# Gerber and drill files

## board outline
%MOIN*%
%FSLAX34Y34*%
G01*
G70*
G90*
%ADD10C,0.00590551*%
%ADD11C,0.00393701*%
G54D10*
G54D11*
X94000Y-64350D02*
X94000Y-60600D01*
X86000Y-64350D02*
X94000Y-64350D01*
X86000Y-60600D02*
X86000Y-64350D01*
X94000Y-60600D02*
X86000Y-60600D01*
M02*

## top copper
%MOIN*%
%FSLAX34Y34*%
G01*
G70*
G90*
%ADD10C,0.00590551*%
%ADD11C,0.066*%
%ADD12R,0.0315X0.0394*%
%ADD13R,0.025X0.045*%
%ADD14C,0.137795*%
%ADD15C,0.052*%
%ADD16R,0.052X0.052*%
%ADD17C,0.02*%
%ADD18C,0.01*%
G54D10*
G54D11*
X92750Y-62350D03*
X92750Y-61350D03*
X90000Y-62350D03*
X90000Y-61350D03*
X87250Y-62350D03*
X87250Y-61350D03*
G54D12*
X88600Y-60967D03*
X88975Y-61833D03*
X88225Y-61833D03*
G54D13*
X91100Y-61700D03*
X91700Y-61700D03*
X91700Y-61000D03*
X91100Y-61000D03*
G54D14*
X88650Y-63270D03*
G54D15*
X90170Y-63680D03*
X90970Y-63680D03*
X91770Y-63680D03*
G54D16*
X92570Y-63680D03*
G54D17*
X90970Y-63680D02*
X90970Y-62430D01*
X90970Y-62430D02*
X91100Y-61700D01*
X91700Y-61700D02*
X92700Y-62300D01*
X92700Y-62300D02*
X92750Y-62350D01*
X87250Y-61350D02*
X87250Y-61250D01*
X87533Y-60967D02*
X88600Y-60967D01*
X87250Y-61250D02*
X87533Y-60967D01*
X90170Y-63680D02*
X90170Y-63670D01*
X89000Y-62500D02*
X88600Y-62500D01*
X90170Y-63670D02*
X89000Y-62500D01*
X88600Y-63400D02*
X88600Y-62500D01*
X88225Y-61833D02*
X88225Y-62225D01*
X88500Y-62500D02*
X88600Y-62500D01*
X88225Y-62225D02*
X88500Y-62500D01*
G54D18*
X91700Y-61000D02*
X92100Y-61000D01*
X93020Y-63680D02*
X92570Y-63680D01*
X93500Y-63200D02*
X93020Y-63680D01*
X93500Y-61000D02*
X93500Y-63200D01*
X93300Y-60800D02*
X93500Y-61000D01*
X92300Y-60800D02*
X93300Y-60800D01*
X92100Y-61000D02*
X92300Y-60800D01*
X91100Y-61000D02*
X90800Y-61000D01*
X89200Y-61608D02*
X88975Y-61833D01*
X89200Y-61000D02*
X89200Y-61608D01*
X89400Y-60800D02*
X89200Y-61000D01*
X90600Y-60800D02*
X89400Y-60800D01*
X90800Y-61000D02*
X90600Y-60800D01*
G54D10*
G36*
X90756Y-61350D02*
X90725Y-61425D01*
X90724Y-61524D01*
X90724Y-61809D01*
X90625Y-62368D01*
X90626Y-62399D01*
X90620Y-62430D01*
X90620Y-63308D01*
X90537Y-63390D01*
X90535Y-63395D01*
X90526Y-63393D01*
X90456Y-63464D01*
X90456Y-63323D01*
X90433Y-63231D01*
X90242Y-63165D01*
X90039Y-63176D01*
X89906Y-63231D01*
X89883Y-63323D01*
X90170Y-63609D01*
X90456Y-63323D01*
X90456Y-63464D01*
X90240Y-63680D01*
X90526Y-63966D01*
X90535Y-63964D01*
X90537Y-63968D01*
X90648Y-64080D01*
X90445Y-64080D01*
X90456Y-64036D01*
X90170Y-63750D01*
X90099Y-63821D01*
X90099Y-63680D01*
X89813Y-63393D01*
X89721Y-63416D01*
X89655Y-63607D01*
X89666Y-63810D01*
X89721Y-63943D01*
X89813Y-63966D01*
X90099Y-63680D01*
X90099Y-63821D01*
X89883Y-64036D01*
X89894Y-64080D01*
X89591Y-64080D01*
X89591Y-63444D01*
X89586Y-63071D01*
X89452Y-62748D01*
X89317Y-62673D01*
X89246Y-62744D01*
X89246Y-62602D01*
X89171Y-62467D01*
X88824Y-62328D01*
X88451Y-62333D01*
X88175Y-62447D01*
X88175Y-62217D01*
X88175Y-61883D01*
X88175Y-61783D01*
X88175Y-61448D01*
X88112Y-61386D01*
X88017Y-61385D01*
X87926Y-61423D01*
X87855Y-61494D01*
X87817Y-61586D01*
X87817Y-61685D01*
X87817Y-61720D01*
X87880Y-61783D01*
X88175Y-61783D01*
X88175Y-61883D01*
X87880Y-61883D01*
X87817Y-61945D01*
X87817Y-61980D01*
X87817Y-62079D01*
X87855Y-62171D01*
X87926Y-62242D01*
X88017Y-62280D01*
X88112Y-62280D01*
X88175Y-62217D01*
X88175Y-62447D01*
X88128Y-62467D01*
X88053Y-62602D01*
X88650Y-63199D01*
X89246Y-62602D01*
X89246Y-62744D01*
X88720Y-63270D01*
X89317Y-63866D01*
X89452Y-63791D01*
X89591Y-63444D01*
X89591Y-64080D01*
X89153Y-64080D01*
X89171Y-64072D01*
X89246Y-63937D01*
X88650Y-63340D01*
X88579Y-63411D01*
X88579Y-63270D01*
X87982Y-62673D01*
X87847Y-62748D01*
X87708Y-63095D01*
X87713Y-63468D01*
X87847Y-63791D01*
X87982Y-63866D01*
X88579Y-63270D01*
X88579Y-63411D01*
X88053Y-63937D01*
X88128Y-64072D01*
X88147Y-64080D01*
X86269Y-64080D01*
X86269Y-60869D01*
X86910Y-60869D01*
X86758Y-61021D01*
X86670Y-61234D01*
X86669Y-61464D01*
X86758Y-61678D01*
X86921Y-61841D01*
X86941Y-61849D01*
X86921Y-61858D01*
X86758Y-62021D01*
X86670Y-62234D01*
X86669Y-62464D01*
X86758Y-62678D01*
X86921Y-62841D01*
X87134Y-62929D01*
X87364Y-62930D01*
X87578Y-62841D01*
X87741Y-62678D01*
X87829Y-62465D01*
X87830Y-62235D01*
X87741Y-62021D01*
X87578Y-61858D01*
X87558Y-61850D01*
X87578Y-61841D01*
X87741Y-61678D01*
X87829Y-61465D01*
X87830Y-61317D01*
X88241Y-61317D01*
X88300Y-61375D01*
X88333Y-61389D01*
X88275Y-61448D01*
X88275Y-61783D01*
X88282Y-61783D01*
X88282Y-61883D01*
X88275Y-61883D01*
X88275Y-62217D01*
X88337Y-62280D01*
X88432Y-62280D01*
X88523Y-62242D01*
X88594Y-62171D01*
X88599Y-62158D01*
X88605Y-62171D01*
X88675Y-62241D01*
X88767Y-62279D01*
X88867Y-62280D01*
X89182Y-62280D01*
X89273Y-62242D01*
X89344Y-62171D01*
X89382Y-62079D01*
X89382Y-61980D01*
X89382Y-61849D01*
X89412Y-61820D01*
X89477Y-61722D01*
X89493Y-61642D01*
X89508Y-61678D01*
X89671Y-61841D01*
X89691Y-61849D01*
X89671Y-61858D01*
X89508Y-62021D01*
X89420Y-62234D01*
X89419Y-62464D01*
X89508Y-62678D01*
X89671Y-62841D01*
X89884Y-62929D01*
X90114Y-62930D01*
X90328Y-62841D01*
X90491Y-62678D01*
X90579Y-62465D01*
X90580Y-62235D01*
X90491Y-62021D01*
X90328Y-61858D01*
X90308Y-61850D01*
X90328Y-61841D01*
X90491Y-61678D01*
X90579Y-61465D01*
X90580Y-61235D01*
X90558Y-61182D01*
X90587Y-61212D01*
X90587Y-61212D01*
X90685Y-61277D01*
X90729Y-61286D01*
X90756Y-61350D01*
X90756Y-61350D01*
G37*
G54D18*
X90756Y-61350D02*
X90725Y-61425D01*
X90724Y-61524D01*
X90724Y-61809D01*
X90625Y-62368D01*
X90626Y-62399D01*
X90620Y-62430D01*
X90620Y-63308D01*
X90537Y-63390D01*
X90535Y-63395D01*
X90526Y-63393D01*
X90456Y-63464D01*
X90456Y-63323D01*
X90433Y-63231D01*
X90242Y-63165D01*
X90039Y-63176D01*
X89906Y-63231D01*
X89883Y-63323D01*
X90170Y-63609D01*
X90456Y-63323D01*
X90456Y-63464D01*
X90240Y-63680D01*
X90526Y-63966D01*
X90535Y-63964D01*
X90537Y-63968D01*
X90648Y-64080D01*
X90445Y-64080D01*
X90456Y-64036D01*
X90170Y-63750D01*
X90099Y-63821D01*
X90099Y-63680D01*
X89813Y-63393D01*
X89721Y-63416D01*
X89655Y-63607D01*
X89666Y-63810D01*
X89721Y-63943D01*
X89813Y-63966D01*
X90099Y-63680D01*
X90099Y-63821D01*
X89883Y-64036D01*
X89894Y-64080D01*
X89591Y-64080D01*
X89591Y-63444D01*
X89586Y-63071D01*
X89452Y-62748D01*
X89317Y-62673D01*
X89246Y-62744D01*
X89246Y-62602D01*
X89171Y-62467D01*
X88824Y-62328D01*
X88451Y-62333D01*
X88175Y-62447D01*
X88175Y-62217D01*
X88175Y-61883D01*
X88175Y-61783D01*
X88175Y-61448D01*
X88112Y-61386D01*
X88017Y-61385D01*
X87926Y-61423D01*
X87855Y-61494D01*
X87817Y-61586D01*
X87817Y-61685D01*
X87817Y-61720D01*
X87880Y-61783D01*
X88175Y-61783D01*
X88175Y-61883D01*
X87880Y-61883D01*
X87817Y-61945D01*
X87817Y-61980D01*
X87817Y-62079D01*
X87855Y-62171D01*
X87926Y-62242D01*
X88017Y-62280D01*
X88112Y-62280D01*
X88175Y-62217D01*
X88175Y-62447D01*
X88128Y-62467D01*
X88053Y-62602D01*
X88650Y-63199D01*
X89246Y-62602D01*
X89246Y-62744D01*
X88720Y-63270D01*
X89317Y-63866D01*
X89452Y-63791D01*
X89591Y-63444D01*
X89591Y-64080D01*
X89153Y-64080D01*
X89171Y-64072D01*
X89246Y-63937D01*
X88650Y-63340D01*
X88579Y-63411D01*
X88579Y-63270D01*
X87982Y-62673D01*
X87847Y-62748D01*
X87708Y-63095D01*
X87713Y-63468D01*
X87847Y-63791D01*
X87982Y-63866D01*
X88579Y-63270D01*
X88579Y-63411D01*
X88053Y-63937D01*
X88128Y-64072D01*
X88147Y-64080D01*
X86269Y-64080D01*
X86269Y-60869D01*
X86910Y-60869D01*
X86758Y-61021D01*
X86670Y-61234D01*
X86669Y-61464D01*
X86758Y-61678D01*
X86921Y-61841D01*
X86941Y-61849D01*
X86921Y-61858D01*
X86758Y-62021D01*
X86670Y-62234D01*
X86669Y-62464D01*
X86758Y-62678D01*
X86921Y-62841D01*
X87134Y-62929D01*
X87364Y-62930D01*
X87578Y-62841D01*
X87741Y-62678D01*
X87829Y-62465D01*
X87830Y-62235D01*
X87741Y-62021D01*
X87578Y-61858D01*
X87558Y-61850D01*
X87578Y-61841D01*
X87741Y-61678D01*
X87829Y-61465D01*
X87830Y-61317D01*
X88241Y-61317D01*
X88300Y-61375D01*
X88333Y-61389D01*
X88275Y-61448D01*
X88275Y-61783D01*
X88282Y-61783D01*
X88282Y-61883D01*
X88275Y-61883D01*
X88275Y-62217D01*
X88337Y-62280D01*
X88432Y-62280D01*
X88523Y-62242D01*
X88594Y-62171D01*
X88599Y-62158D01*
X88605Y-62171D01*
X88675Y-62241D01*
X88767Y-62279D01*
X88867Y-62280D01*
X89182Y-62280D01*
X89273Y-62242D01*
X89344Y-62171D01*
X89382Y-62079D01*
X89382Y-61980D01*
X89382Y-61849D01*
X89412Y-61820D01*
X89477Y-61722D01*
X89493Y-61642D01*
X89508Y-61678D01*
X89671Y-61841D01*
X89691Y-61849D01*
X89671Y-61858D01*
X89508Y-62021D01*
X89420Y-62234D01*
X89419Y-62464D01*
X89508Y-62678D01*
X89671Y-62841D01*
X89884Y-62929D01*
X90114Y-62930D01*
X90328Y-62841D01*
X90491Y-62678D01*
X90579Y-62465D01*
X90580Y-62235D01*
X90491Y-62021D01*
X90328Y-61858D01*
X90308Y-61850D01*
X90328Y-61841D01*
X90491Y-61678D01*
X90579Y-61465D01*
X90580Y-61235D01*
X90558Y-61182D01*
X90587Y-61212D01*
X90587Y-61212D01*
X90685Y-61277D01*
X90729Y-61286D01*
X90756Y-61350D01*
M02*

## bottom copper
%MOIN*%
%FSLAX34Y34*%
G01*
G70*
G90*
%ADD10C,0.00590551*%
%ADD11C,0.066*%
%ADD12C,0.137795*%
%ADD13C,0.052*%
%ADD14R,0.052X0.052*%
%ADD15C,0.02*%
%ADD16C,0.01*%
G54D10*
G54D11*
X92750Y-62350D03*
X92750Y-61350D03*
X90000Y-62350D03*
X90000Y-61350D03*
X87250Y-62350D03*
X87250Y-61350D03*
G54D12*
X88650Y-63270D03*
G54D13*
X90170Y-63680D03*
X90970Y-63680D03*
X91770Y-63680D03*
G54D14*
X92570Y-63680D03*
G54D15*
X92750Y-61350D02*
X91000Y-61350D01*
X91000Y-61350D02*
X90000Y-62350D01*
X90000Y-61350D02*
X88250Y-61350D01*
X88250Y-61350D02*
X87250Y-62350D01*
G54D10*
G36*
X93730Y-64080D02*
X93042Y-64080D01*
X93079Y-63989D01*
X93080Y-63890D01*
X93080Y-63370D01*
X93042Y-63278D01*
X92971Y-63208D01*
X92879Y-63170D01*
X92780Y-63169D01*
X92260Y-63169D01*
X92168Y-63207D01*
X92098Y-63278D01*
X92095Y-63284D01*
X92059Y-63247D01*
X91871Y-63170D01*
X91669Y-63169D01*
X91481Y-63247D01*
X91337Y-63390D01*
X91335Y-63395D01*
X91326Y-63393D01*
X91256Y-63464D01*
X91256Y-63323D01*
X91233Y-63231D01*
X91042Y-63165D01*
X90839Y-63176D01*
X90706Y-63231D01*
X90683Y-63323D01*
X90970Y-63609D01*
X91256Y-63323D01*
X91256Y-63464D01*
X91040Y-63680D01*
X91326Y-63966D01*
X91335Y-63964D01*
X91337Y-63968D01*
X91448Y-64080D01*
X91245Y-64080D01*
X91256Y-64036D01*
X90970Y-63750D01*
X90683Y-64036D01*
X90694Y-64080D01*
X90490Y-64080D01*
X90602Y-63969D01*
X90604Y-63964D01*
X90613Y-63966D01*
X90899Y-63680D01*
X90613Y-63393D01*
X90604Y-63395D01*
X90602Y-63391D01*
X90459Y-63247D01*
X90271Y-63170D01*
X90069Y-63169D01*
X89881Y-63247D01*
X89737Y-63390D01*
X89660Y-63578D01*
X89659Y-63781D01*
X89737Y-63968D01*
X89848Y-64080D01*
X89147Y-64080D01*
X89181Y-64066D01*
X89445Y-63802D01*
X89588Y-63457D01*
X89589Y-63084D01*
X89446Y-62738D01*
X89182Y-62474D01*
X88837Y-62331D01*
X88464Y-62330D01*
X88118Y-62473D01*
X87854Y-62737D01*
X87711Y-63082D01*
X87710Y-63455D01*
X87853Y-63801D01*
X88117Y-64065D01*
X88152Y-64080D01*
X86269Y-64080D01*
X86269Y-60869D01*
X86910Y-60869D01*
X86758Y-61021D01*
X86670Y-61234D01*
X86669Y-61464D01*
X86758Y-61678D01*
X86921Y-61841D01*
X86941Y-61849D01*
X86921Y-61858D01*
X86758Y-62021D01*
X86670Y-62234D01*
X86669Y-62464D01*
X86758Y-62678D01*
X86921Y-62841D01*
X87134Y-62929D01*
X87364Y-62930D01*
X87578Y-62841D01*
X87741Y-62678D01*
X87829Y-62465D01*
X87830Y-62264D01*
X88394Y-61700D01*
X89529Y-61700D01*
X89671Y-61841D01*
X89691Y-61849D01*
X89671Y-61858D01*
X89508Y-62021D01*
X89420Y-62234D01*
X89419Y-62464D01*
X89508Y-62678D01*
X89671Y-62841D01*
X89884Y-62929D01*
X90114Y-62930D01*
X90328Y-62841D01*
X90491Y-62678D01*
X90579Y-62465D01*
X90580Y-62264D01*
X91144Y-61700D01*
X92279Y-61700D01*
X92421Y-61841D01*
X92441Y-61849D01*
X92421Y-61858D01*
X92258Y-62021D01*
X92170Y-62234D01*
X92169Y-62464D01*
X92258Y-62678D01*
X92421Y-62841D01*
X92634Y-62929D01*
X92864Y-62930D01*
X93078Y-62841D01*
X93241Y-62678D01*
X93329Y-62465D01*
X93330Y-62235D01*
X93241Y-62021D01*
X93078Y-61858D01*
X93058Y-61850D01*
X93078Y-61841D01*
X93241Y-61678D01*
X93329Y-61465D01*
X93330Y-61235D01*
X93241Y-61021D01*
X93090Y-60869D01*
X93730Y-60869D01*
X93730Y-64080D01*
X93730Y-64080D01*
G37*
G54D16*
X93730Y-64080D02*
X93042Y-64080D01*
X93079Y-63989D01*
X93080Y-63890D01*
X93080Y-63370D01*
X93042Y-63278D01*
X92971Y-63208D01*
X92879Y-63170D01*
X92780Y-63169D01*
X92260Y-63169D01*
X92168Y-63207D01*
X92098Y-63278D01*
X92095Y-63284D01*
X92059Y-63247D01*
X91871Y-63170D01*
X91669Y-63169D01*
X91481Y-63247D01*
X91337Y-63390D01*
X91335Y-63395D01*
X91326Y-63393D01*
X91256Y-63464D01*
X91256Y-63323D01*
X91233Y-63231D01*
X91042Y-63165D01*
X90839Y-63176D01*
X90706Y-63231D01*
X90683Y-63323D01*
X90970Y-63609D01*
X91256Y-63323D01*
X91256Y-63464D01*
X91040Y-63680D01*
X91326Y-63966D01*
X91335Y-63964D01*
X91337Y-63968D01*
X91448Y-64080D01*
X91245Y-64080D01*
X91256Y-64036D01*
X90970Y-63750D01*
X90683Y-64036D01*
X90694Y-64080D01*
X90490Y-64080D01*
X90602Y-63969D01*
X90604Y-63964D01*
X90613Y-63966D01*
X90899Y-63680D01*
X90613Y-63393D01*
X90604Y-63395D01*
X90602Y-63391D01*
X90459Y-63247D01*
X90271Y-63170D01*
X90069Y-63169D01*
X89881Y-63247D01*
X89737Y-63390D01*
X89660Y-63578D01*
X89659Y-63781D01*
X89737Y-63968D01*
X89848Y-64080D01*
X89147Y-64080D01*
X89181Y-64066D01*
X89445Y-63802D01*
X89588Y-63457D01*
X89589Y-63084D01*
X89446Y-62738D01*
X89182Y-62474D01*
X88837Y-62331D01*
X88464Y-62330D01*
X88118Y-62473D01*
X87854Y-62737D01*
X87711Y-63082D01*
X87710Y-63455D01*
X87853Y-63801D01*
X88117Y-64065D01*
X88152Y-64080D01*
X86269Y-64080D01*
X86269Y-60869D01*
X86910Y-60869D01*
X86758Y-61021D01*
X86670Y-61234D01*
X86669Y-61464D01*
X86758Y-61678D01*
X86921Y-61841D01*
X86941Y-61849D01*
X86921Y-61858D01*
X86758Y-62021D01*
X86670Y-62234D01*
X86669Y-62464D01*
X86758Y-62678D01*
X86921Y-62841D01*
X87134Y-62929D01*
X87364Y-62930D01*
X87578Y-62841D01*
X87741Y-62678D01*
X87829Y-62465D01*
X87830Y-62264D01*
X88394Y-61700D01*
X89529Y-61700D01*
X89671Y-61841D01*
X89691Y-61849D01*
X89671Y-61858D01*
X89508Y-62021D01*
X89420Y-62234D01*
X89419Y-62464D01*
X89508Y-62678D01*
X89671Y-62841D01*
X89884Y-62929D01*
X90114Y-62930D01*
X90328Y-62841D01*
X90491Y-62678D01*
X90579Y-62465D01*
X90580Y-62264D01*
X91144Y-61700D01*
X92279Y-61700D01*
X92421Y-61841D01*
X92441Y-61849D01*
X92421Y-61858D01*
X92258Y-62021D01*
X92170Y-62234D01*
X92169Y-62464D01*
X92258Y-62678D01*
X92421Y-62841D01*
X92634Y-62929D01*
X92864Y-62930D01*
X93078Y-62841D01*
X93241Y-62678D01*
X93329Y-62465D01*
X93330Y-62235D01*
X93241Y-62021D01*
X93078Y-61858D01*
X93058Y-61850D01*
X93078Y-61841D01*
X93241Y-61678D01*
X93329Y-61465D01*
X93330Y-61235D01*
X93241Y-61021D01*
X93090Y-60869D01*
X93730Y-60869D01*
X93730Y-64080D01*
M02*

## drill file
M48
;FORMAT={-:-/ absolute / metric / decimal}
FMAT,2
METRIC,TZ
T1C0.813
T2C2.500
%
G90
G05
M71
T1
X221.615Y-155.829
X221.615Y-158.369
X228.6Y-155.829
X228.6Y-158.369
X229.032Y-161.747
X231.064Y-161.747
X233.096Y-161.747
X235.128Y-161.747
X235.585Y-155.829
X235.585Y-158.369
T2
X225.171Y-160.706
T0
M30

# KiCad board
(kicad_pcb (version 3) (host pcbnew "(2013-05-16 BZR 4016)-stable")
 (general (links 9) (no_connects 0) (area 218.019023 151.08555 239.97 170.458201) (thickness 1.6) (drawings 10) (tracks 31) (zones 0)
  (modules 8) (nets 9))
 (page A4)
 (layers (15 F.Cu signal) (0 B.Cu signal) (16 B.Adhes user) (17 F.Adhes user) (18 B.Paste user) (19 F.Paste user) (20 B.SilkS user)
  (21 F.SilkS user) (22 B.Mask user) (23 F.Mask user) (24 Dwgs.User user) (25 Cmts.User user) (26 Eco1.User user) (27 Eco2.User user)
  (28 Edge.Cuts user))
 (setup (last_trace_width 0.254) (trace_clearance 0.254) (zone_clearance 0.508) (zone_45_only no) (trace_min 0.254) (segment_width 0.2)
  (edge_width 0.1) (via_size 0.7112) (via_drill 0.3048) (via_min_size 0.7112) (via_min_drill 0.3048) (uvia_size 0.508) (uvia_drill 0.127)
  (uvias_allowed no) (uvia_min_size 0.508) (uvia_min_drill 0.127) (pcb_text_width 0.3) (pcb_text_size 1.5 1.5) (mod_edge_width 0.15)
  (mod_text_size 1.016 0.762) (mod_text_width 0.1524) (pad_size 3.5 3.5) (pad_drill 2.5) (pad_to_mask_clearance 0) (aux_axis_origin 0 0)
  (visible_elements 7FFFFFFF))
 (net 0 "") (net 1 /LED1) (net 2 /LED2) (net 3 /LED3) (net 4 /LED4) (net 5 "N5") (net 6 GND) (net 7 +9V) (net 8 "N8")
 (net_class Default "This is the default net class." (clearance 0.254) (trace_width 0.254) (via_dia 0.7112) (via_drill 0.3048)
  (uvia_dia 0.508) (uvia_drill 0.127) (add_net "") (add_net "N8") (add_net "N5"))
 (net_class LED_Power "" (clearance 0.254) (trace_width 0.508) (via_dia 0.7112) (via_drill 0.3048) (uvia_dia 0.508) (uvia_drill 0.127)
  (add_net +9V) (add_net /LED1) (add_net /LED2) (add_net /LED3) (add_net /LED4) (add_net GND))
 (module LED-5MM (layer B.Cu) (at 235.585 157.099 90)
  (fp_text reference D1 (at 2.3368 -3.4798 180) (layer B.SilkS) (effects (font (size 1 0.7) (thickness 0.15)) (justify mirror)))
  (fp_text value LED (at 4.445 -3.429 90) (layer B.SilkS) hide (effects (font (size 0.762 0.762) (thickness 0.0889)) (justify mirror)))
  (pad 1 thru_hole circle (at -1.27 0 90) (size 1.6764 1.6764) (drill 0.8128) (layers *.Cu *.Mask B.SilkS) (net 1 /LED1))
  (pad 2 thru_hole circle (at 1.27 0 90) (size 1.6764 1.6764) (drill 0.8128) (layers *.Cu *.Mask B.SilkS) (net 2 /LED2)))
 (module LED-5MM (layer B.Cu) (at 228.6 157.099 90)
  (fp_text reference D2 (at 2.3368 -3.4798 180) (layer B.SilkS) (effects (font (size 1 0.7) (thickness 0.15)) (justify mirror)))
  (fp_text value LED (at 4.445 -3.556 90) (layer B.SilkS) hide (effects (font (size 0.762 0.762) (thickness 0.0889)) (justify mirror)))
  (pad 1 thru_hole circle (at -1.27 0 90) (size 1.6764 1.6764) (drill 0.8128) (layers *.Cu *.Mask B.SilkS) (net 2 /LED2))
  (pad 2 thru_hole circle (at 1.27 0 90) (size 1.6764 1.6764) (drill 0.8128) (layers *.Cu *.Mask B.SilkS) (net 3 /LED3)))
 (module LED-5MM (layer B.Cu) (at 221.615 157.099 90)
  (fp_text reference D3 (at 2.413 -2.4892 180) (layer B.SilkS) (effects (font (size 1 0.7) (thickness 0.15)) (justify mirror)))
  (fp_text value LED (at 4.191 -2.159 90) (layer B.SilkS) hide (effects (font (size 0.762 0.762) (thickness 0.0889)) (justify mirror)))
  (pad 1 thru_hole circle (at -1.27 0 90) (size 1.6764 1.6764) (drill 0.8128) (layers *.Cu *.Mask B.SilkS) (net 3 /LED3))
  (pad 2 thru_hole circle (at 1.27 0 90) (size 1.6764 1.6764) (drill 0.8128) (layers *.Cu *.Mask B.SilkS) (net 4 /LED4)))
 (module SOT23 (layer F.Cu) (at 225.044 155.956)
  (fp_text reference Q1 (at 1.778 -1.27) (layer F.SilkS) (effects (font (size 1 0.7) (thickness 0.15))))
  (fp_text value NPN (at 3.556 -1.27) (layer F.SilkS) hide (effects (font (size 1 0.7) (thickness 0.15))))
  (pad 3 smd rect (at 0 -1.09982) (size 0.8001 1.00076) (layers F.Cu F.Paste F.Mask) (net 4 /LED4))
  (pad 2 smd rect (at 0.9525 1.09982) (size 0.8001 1.00076) (layers F.Cu F.Paste F.Mask) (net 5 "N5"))
  (pad 1 smd rect (at -0.9525 1.09982) (size 0.8001 1.00076) (layers F.Cu F.Paste F.Mask) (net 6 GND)))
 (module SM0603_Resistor (layer F.Cu) (at 232.156 156.718)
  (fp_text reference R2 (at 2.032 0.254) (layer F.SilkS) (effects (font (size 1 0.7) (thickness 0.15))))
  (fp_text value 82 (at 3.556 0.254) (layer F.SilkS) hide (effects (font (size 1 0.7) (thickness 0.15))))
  (pad 1 smd rect (at -0.762 0) (size 0.635 1.143) (layers F.Cu F.Paste F.Mask) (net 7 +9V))
  (pad 2 smd rect (at 0.762 0) (size 0.635 1.143) (layers F.Cu F.Paste F.Mask) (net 1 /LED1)))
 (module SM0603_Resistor (layer F.Cu) (at 232.156 154.94 180)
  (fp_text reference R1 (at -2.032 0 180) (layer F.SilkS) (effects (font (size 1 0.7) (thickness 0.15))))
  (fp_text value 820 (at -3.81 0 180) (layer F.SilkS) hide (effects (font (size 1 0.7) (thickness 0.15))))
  (pad 1 smd rect (at -0.762 0 180) (size 0.635 1.143) (layers F.Cu F.Paste F.Mask) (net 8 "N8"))
  (pad 2 smd rect (at 0.762 0 180) (size 0.635 1.143) (layers F.Cu F.Paste F.Mask) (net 5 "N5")))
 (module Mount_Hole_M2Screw (layer F.Cu) (at 225.171 160.7058)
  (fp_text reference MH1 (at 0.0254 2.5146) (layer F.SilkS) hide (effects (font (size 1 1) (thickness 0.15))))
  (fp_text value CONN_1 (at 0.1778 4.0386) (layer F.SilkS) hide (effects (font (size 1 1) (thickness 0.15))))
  (pad 1 thru_hole circle (at 0 0) (size 3.5 3.5) (drill 2.5) (layers *.Cu *.Mask F.SilkS) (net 6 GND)))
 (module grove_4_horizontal (layer F.Cu) (at 227.076 160.274 90)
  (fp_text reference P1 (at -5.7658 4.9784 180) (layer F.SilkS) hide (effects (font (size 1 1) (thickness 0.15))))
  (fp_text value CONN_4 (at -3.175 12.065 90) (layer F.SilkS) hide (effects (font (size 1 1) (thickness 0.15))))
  (pad 4 thru_hole circle (at -1.4732 1.9558 90) (size 1.3208 1.3208) (drill 0.8128) (layers *.Cu *.Mask F.SilkS) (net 6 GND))
  (pad 3 thru_hole circle (at -1.4732 3.9878 90) (size 1.3208 1.3208) (drill 0.8128) (layers *.Cu *.Mask F.SilkS) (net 7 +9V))
  (pad 2 thru_hole circle (at -1.4732 6.0198 90) (size 1.3208 1.3208) (drill 0.8128) (layers *.Cu *.Mask F.SilkS))
  (pad 1 thru_hole rect (at -1.4732 8.0518 90) (size 1.3208 1.3208) (drill 0.8128) (layers *.Cu *.Mask F.SilkS) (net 8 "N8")))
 (gr_line (start 238.76 163.449) (end 238.76 153.924) (angle 90) (layer Edge.Cuts) (width 0.1))
 (gr_line (start 218.44 163.449) (end 238.76 163.449) (angle 90) (layer Edge.Cuts) (width 0.1))
 (gr_line (start 218.44 153.924) (end 218.44 163.449) (angle 90) (layer Edge.Cuts) (width 0.1))
 (gr_line (start 238.76 153.924) (end 218.44 153.924) (angle 90) (layer Edge.Cuts) (width 0.1))
 (segment (start 231.0638 161.7472) (end 231.0638 158.5722) (width 0.508) (layer F.Cu) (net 7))
 (segment (start 231.0638 158.5722) (end 231.394 156.718) (width 0.508) (layer F.Cu) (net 7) (status 20))
 (segment (start 232.918 156.718) (end 235.458 158.242) (width 0.508) (layer F.Cu) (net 1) (status 10))
 (segment (start 235.458 158.242) (end 235.585 158.369) (width 0.508) (layer F.Cu) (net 1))
 (segment (start 235.585 155.829) (end 231.14 155.829) (width 0.508) (layer B.Cu) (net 2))
 (segment (start 231.14 155.829) (end 228.6 158.369) (width 0.508) (layer B.Cu) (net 2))
 (segment (start 228.6 155.829) (end 224.155 155.829) (width 0.508) (layer B.Cu) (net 3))
 (segment (start 224.155 155.829) (end 221.615 158.369) (width 0.508) (layer B.Cu) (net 3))
 (segment (start 221.615 155.829) (end 221.615 155.575) (width 0.508) (layer F.Cu) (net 4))
 (segment (start 222.33382 154.85618) (end 225.044 154.85618) (width 0.508) (layer F.Cu) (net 4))
 (segment (start 221.615 155.575) (end 222.33382 154.85618) (width 0.508) (layer F.Cu) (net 4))
 (segment (start 229.0318 161.7472) (end 229.0318 161.7218) (width 0.508) (layer F.Cu) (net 6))
 (segment (start 226.06 158.75) (end 225.044 158.75) (width 0.508) (layer F.Cu) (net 6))
 (segment (start 229.0318 161.7218) (end 226.06 158.75) (width 0.508) (layer F.Cu) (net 6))
 (segment (start 225.044 161.036) (end 225.044 158.75) (width 0.508) (layer F.Cu) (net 6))
 (segment (start 224.0915 157.05582) (end 224.0915 158.0515) (width 0.508) (layer F.Cu) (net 6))
 (segment (start 224.79 158.75) (end 225.044 158.75) (width 0.508) (layer F.Cu) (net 6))
 (segment (start 224.0915 158.0515) (end 224.79 158.75) (width 0.508) (layer F.Cu) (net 6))
 (segment (start 232.918 154.94) (end 233.934 154.94) (width 0.254) (layer F.Cu) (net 8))
 (segment (start 236.2708 161.7472) (end 235.1278 161.7472) (width 0.254) (layer F.Cu) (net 8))
 (segment (start 237.49 160.528) (end 236.2708 161.7472) (width 0.254) (layer F.Cu) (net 8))
 (segment (start 237.49 154.94) (end 237.49 160.528) (width 0.254) (layer F.Cu) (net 8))
 (segment (start 236.982 154.432) (end 237.49 154.94) (width 0.254) (layer F.Cu) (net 8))
 (segment (start 234.442 154.432) (end 236.982 154.432) (width 0.254) (layer F.Cu) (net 8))
 (segment (start 233.934 154.94) (end 234.442 154.432) (width 0.254) (layer F.Cu) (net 8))
 (segment (start 231.394 154.94) (end 230.632 154.94) (width 0.254) (layer F.Cu) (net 5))
 (segment (start 226.568 156.48432) (end 225.9965 157.05582) (width 0.254) (layer F.Cu) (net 5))
 (segment (start 226.568 154.94) (end 226.568 156.48432) (width 0.254) (layer F.Cu) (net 5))
 (segment (start 227.076 154.432) (end 226.568 154.94) (width 0.254) (layer F.Cu) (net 5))
 (segment (start 230.124 154.432) (end 227.076 154.432) (width 0.254) (layer F.Cu) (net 5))
 (segment (start 230.632 154.94) (end 230.124 154.432) (width 0.254) (layer F.Cu) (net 5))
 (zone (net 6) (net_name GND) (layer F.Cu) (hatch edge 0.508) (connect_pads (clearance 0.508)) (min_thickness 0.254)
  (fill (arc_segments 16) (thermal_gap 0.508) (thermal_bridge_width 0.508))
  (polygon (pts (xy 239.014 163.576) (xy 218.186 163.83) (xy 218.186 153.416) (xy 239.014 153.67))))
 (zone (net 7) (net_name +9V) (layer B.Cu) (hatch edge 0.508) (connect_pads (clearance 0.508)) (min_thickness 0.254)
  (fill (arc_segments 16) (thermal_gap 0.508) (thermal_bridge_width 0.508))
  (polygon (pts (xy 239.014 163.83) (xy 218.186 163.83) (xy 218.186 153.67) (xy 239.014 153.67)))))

